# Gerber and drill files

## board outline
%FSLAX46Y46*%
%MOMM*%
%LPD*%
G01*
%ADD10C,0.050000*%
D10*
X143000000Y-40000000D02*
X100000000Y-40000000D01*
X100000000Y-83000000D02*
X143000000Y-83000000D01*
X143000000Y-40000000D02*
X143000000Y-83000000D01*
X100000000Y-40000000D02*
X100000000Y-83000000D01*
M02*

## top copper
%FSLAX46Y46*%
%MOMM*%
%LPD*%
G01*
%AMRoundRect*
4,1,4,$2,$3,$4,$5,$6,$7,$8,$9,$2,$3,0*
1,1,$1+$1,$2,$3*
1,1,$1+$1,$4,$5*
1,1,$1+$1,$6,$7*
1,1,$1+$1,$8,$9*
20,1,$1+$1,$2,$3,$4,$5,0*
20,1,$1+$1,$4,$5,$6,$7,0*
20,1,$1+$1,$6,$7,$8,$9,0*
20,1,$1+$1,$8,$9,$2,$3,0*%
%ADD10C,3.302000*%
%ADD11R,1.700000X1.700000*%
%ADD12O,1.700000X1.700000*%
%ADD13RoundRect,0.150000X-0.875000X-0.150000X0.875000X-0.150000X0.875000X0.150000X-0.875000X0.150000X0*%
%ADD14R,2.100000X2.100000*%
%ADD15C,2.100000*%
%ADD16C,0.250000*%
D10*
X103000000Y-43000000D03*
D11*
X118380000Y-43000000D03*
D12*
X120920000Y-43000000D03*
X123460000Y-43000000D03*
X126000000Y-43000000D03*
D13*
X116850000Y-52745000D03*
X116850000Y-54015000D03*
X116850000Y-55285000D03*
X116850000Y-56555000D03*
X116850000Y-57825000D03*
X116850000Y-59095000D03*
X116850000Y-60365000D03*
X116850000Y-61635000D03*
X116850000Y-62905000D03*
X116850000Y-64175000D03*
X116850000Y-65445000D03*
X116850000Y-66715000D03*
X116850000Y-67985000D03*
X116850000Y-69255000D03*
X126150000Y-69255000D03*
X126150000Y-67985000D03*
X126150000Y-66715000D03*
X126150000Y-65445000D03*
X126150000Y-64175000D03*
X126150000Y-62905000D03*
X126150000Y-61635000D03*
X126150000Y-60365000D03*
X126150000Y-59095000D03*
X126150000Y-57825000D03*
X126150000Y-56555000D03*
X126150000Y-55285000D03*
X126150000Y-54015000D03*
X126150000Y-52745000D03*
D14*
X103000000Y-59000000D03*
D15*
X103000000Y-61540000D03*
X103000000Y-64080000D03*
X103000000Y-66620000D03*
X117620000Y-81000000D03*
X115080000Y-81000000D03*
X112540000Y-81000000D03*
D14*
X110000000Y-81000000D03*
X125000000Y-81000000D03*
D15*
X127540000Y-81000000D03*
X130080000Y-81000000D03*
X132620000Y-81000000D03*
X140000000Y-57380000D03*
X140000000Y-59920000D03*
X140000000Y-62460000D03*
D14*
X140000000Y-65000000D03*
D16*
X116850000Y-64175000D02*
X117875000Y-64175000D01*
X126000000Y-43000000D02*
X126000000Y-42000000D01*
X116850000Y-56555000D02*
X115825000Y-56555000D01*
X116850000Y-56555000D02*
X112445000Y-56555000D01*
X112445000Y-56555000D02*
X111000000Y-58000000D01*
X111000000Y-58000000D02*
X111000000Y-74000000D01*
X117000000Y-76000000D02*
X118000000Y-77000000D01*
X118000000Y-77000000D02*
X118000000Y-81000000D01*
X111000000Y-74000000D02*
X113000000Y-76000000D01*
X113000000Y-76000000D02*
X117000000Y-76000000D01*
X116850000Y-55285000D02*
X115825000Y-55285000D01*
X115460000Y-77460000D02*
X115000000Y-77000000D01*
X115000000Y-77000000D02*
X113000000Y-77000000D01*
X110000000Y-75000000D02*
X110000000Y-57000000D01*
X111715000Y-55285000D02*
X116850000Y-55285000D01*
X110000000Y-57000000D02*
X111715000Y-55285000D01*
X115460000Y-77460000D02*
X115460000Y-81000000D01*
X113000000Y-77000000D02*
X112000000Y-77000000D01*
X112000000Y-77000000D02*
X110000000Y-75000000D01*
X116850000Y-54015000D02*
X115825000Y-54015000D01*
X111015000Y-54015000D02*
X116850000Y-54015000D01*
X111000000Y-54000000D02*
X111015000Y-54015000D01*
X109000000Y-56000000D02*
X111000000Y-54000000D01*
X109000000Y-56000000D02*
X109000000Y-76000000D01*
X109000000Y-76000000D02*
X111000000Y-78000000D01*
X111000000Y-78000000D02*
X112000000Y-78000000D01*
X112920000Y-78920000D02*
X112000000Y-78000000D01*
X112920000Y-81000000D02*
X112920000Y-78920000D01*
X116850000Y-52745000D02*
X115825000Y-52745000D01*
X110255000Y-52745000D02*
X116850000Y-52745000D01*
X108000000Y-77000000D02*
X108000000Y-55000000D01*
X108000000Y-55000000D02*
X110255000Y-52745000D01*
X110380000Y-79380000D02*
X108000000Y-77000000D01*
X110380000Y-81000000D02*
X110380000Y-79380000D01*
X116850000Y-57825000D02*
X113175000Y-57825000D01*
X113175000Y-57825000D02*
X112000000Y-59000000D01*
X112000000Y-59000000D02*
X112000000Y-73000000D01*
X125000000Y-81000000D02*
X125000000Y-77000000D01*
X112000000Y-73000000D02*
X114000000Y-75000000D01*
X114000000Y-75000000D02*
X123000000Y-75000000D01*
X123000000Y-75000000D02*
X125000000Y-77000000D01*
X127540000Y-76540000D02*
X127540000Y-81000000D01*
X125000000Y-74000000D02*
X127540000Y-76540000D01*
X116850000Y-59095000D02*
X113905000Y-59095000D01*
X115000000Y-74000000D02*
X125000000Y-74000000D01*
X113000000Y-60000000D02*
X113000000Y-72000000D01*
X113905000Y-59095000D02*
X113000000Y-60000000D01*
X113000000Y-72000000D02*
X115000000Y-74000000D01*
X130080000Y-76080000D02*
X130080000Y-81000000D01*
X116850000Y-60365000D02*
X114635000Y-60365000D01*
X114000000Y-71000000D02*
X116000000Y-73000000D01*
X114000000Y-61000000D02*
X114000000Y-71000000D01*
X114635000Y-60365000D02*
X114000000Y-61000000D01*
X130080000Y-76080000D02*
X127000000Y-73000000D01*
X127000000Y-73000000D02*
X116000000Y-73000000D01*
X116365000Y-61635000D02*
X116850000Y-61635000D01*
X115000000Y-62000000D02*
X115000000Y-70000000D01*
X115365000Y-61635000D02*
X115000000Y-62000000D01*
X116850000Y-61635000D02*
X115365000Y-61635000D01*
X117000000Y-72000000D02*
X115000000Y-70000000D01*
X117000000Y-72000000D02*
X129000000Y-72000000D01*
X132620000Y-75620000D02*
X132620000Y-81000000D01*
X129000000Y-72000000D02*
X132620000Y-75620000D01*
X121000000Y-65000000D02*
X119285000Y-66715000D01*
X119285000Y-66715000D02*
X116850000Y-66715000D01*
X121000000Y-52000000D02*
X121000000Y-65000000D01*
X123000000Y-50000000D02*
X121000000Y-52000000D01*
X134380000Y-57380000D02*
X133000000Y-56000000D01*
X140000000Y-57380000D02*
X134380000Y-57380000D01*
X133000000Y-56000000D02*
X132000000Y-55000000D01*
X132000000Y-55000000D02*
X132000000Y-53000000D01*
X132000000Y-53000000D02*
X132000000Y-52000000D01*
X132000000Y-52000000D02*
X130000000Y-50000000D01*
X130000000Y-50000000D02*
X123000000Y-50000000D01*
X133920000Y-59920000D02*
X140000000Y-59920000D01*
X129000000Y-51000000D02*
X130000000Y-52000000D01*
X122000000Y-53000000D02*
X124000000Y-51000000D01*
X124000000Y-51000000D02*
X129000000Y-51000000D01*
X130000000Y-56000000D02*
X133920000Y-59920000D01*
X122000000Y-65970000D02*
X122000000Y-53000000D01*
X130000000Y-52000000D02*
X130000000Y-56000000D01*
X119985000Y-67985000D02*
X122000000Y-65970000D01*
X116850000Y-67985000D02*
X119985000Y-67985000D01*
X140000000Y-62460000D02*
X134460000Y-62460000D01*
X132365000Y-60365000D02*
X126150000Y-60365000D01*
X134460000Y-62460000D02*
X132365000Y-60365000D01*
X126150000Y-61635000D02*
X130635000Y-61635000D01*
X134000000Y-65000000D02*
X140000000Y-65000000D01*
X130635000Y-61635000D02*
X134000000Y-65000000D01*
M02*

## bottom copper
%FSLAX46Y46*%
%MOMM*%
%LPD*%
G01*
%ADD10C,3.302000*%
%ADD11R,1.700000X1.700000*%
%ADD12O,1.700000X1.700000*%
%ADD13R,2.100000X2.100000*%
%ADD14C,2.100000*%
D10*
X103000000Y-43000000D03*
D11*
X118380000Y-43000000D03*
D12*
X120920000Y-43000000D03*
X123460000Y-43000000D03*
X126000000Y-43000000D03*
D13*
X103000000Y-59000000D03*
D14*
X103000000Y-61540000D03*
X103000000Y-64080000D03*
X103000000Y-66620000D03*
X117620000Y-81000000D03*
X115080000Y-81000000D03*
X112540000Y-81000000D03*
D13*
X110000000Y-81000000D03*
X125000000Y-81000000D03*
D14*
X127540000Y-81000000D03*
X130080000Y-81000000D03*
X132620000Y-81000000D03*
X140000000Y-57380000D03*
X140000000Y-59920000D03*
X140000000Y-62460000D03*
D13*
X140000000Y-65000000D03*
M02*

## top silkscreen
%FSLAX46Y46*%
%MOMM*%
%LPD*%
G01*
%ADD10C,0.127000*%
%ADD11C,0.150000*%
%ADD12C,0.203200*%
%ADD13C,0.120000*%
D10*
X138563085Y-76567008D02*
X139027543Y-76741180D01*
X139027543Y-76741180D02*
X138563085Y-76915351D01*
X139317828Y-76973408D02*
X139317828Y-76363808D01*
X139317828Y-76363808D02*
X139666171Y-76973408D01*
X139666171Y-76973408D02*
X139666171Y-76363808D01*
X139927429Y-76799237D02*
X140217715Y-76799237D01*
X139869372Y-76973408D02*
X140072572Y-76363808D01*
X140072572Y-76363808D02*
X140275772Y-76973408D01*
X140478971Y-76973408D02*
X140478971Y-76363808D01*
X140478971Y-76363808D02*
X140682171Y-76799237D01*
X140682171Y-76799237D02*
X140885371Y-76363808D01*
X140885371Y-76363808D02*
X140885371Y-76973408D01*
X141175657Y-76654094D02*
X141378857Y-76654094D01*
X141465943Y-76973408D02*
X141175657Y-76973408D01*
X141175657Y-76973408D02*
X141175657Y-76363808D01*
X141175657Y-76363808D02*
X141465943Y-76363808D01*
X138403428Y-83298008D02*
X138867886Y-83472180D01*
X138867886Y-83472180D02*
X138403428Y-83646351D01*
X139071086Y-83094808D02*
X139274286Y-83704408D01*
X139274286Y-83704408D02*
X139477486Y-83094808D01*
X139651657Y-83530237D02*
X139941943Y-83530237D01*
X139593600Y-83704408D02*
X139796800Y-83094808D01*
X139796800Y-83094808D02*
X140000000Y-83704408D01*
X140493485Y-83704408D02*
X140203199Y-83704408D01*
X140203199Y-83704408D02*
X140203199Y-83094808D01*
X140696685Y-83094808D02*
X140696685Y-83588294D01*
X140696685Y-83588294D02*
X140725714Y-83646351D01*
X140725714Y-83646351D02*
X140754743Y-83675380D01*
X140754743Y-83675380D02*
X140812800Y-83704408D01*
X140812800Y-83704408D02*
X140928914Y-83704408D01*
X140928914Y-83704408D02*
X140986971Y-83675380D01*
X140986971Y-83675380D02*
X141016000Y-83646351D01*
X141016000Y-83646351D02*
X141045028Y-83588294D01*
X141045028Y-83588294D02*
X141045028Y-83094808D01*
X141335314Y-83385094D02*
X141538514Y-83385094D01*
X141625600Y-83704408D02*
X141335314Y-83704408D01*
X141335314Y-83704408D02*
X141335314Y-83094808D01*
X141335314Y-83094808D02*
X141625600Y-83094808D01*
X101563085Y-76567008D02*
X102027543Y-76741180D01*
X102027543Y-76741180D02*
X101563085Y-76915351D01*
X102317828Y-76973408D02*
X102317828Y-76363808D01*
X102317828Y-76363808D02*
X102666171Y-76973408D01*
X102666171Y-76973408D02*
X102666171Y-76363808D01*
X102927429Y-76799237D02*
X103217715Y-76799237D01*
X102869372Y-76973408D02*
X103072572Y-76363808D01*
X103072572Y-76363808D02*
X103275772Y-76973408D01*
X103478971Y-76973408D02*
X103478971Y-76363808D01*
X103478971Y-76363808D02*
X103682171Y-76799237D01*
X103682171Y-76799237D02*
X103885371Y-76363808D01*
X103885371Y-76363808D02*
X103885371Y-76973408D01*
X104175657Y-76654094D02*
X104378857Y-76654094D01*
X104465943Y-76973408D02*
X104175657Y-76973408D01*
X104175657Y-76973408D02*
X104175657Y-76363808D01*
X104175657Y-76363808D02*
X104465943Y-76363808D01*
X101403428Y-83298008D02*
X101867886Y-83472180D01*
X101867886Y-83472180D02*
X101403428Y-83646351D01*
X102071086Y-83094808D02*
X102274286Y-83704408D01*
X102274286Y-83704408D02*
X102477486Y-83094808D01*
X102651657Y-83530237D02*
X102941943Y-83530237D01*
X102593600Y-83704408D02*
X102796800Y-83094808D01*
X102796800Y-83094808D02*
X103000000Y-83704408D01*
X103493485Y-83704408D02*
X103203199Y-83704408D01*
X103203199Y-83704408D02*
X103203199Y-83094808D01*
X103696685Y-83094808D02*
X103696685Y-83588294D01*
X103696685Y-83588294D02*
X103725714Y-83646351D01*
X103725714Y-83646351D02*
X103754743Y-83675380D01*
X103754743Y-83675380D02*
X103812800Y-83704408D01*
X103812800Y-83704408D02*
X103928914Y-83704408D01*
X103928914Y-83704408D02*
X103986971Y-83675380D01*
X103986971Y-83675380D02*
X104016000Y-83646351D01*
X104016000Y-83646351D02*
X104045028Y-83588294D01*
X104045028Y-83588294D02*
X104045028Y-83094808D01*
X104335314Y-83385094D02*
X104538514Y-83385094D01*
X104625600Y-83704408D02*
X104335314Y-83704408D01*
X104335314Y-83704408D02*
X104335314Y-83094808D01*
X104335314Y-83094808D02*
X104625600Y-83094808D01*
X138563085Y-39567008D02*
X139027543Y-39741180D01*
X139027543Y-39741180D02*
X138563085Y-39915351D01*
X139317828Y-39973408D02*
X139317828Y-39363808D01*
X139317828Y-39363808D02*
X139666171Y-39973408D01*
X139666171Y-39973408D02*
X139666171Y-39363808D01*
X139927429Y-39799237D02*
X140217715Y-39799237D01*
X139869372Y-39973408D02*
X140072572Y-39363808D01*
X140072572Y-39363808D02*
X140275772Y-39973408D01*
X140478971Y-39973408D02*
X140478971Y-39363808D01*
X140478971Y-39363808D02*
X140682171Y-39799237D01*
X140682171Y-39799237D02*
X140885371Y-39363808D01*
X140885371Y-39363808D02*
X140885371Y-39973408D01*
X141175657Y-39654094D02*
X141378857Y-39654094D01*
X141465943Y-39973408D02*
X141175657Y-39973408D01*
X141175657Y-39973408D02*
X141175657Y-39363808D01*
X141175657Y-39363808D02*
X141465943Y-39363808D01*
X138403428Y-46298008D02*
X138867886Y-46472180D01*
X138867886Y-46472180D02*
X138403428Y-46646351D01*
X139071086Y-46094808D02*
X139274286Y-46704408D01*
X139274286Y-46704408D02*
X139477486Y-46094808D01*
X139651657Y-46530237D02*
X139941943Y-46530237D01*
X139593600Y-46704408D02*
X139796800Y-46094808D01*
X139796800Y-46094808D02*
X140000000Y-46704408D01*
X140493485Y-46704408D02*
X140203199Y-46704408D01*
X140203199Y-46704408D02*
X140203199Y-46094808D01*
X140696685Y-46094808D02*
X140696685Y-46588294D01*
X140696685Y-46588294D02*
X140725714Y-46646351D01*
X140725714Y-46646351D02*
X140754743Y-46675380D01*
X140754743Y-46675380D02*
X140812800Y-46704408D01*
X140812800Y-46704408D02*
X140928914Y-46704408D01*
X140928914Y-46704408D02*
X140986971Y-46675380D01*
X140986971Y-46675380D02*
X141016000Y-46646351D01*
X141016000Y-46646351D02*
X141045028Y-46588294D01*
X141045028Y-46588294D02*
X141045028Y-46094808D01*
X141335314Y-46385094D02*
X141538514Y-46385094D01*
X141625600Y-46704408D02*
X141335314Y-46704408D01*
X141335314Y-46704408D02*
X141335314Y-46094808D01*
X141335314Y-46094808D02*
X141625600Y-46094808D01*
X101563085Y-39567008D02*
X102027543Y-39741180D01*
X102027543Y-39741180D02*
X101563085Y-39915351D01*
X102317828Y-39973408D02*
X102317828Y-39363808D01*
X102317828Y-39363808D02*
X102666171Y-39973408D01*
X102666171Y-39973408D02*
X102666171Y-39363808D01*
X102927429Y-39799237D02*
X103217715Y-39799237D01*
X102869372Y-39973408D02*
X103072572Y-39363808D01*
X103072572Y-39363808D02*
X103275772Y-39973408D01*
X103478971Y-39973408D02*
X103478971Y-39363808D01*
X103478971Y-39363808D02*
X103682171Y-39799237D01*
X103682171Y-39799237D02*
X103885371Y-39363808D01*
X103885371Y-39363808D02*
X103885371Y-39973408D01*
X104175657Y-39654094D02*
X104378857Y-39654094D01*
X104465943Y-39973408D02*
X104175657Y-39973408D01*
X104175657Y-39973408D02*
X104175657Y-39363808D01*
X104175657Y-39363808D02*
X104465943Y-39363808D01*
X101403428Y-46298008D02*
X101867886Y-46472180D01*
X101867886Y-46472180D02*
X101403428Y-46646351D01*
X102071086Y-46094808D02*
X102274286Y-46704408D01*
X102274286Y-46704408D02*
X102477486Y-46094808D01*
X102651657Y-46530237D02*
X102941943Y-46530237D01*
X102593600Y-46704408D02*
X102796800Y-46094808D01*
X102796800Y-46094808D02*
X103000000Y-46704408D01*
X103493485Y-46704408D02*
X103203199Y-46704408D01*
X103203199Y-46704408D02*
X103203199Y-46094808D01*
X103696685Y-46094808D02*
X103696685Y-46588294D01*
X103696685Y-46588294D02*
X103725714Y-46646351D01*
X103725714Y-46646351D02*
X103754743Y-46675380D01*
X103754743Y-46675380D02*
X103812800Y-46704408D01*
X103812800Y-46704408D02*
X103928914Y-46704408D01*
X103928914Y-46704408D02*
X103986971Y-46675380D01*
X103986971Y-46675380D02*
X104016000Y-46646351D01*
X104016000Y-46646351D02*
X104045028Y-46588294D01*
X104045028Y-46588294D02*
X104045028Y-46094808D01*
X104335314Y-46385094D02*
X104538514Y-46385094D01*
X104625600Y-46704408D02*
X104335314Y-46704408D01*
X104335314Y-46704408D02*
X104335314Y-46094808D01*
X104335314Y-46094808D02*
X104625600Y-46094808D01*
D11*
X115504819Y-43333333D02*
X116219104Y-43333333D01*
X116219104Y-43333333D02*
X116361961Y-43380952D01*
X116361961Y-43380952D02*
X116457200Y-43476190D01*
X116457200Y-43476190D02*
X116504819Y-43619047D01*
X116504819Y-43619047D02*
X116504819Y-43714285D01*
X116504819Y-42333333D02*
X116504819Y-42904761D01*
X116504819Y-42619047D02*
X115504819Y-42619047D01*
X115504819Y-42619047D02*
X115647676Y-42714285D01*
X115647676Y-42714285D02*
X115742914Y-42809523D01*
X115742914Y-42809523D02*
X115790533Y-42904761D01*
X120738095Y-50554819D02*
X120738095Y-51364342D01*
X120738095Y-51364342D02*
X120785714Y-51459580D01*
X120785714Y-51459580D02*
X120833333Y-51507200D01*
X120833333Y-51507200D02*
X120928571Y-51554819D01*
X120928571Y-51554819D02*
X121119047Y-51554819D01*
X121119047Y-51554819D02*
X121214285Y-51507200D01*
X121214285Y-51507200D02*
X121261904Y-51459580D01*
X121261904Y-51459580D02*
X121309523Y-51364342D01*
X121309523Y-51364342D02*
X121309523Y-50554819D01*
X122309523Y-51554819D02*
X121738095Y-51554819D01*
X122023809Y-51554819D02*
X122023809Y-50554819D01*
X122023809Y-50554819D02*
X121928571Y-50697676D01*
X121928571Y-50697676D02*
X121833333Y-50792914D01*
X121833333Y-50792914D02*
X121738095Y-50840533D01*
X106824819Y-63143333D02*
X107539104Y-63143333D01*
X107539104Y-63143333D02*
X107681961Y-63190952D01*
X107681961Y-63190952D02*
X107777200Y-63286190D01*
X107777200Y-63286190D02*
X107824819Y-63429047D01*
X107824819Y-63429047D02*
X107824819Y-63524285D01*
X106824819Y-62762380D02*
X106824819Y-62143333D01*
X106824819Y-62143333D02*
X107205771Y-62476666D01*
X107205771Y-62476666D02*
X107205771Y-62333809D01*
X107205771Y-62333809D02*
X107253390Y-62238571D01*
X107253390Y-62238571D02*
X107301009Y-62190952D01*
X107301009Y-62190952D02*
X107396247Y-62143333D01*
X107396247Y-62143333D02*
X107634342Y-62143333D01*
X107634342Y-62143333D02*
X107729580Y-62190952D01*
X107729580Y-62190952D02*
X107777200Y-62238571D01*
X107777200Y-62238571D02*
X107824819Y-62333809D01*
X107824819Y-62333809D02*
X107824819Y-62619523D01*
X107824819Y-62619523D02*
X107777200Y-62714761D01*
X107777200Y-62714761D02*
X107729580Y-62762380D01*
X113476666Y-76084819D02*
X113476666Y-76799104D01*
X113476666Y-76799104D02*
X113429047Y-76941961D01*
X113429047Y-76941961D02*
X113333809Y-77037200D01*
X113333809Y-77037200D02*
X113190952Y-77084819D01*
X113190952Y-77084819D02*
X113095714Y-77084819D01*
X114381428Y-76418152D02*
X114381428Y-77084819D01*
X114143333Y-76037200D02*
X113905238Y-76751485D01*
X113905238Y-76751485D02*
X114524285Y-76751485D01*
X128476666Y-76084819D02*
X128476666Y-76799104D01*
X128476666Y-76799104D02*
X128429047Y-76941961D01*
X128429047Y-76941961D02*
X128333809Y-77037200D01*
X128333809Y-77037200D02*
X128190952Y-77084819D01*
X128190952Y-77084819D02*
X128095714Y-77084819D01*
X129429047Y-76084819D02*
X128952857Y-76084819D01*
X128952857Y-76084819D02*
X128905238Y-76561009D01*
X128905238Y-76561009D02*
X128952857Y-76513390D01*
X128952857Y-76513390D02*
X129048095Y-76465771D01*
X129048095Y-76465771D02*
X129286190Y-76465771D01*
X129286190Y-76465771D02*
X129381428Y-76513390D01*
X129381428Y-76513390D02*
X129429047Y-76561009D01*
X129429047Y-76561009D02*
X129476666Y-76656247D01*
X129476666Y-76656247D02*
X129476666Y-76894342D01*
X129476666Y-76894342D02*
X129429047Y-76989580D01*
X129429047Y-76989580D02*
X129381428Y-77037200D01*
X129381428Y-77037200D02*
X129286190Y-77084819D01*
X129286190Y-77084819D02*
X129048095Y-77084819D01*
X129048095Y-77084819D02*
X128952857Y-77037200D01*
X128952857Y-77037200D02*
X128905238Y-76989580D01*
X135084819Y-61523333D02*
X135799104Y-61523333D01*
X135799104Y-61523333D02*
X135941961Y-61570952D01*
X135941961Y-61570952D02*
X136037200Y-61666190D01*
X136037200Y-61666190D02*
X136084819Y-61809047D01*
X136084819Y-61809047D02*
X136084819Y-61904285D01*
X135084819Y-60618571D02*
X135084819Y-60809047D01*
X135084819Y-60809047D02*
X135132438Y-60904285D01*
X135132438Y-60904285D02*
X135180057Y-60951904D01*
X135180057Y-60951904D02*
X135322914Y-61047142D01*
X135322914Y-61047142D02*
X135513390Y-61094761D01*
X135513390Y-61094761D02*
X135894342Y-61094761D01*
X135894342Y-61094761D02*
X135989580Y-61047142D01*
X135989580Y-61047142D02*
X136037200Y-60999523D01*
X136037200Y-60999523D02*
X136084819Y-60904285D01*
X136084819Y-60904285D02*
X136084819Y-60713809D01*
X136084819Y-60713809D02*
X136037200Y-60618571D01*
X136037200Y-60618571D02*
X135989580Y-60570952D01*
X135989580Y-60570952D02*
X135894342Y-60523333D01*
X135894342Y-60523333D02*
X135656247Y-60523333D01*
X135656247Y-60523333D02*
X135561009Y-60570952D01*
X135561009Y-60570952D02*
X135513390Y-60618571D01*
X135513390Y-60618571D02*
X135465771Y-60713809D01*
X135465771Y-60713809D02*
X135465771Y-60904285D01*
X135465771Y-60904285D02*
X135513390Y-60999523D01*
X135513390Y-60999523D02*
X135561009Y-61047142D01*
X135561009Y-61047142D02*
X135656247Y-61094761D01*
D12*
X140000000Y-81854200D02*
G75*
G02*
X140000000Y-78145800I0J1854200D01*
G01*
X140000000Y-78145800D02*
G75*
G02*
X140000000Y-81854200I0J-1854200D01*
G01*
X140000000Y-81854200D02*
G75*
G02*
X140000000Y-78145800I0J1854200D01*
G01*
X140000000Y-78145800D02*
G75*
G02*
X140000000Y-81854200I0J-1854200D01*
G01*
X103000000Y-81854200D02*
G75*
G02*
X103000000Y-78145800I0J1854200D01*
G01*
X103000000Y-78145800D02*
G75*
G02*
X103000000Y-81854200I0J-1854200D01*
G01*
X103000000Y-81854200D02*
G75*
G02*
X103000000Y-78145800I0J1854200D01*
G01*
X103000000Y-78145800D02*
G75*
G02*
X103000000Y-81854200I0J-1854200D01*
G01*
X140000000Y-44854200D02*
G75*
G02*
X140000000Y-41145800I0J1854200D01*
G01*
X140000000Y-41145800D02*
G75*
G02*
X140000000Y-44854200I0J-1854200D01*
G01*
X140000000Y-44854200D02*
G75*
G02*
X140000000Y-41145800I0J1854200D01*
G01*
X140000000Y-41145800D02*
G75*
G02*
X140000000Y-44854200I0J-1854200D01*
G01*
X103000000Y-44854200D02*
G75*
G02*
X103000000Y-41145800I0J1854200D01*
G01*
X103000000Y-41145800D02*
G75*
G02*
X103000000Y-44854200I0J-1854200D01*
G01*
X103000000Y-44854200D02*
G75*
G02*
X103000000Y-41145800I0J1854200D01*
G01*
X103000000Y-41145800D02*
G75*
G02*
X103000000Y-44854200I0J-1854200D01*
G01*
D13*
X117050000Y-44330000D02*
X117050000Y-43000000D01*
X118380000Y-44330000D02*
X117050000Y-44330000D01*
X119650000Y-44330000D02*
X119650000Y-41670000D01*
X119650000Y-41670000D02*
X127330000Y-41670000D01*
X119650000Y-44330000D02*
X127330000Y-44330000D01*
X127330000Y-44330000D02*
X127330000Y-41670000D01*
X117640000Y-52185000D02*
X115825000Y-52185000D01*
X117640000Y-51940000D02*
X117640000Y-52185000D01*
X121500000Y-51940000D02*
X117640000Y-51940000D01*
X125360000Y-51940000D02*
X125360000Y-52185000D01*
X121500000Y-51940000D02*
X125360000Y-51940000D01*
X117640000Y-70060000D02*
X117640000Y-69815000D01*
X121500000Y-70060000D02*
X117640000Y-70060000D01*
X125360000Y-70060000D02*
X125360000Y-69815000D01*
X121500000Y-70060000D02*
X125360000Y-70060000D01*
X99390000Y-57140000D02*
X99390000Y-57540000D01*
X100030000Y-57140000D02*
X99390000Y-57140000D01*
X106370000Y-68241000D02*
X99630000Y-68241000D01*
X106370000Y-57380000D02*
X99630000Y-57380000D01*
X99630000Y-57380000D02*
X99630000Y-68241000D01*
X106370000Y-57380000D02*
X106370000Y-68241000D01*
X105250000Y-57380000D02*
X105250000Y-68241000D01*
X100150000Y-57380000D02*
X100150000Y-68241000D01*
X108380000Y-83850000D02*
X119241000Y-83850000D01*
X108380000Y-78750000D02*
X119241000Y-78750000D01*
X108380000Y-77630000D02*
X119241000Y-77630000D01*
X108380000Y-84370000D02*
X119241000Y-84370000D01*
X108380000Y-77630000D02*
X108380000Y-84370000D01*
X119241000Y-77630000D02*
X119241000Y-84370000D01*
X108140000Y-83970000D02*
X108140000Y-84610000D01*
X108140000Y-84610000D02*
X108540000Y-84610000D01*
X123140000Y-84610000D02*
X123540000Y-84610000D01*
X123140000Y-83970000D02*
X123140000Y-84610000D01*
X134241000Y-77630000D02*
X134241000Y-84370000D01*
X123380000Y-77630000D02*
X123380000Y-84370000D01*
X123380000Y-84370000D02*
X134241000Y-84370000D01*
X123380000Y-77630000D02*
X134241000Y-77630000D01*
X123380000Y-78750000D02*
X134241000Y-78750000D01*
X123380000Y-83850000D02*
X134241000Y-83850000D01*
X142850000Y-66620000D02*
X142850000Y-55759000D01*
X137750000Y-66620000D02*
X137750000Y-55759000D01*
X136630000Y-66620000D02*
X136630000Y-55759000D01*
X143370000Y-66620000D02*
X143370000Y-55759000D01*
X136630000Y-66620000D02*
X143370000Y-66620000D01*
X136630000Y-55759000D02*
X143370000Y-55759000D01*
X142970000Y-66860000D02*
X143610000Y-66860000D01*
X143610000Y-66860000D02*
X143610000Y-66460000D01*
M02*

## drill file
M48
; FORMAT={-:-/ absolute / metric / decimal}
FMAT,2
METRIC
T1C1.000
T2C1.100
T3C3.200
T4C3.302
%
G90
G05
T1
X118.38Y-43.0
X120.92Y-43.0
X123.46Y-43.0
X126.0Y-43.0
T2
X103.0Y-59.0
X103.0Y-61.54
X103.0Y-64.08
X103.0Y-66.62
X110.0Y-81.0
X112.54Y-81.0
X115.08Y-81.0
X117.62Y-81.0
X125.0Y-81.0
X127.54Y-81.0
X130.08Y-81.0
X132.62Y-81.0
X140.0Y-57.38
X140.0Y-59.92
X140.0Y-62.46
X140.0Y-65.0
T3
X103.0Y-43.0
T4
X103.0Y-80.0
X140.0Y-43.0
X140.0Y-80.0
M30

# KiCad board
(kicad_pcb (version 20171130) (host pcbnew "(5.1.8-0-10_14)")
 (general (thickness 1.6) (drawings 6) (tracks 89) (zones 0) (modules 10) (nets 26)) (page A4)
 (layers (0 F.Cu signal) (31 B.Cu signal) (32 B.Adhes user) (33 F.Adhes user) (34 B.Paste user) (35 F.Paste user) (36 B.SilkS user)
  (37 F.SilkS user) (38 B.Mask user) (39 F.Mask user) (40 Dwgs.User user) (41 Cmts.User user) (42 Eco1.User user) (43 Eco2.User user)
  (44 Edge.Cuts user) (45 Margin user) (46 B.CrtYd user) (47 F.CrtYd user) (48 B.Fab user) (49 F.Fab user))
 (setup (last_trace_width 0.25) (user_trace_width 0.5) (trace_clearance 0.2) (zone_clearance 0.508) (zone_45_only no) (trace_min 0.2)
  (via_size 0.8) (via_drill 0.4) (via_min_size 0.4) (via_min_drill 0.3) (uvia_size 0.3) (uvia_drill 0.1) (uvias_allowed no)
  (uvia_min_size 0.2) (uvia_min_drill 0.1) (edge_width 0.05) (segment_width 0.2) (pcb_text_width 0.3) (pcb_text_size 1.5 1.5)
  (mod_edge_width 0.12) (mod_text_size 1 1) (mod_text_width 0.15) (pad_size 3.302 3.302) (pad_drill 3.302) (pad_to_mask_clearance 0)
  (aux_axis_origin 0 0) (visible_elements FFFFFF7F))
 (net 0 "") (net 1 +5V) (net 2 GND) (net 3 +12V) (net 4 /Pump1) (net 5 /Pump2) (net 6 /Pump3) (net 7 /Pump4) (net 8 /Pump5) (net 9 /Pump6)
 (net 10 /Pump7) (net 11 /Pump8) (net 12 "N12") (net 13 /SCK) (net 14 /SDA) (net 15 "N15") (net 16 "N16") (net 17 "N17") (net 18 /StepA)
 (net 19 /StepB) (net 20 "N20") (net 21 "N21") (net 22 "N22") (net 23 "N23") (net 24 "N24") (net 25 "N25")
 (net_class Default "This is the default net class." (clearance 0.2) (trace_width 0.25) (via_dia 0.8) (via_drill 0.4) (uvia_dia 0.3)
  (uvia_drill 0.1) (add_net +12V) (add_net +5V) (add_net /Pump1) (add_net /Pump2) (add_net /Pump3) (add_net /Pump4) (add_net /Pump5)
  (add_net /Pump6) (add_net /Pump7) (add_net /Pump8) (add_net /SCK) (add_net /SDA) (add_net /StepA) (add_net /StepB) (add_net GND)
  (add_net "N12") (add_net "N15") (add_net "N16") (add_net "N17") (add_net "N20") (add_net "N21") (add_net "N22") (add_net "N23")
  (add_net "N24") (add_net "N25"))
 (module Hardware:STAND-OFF (layer F.Cu) (at 140 80)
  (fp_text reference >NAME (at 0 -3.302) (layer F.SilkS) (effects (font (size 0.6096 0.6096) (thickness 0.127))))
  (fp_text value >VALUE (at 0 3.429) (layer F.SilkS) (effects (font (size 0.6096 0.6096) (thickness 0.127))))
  (fp_arc (start 0 0) (end 0 1.8542) (angle 180) (layer F.SilkS) (width 0.2032))
  (fp_arc (start 0 0) (end 0 -1.8542) (angle 180) (layer F.SilkS) (width 0.2032))
  (fp_arc (start 0 0) (end 0 1.8542) (angle 180) (layer F.SilkS) (width 0.2032))
  (fp_arc (start 0 0) (end 0 -1.8542) (angle 180) (layer F.SilkS) (width 0.2032))
  (pad "" np_thru_hole circle (at 0 0) (size 3.302 3.302) (drill 3.302) (layers *.Cu *.Mask) (solder_mask_margin 0.1016)))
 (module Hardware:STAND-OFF (layer F.Cu) (at 103 80)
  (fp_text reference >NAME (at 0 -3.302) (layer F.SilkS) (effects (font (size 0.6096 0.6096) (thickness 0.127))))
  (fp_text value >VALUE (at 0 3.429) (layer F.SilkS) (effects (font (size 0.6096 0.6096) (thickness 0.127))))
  (fp_arc (start 0 0) (end 0 1.8542) (angle 180) (layer F.SilkS) (width 0.2032))
  (fp_arc (start 0 0) (end 0 -1.8542) (angle 180) (layer F.SilkS) (width 0.2032))
  (fp_arc (start 0 0) (end 0 1.8542) (angle 180) (layer F.SilkS) (width 0.2032))
  (fp_arc (start 0 0) (end 0 -1.8542) (angle 180) (layer F.SilkS) (width 0.2032))
  (pad "" np_thru_hole circle (at 0 0) (size 3.302 3.302) (drill 3.302) (layers *.Cu *.Mask) (solder_mask_margin 0.1016)))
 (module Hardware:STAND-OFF (layer F.Cu) (at 140 43)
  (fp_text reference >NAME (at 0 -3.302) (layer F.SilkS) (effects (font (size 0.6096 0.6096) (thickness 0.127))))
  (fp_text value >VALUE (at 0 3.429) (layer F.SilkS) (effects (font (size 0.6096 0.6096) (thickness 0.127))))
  (fp_arc (start 0 0) (end 0 1.8542) (angle 180) (layer F.SilkS) (width 0.2032))
  (fp_arc (start 0 0) (end 0 -1.8542) (angle 180) (layer F.SilkS) (width 0.2032))
  (fp_arc (start 0 0) (end 0 1.8542) (angle 180) (layer F.SilkS) (width 0.2032))
  (fp_arc (start 0 0) (end 0 -1.8542) (angle 180) (layer F.SilkS) (width 0.2032))
  (pad "" np_thru_hole circle (at 0 0) (size 3.302 3.302) (drill 3.302) (layers *.Cu *.Mask) (solder_mask_margin 0.1016)))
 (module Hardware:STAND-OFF (layer F.Cu) (at 103 43)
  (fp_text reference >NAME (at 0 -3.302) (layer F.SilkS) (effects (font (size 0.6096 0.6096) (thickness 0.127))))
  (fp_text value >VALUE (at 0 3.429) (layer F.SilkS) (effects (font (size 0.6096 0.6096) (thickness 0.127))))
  (fp_arc (start 0 0) (end 0 1.8542) (angle 180) (layer F.SilkS) (width 0.2032))
  (fp_arc (start 0 0) (end 0 -1.8542) (angle 180) (layer F.SilkS) (width 0.2032))
  (fp_arc (start 0 0) (end 0 1.8542) (angle 180) (layer F.SilkS) (width 0.2032))
  (fp_arc (start 0 0) (end 0 -1.8542) (angle 180) (layer F.SilkS) (width 0.2032))
  (pad "" np_thru_hole circle (at 0 0) (size 3.302 3.302) (drill 3.2) (layers *.Cu *.Mask) (solder_mask_margin 0.1016)))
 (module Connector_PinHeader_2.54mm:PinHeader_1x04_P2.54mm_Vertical (layer F.Cu) (at 118.38 43 90)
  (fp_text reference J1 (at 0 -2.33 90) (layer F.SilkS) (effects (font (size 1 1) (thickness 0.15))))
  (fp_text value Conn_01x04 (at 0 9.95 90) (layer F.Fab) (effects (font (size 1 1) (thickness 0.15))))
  (fp_line (start -1.33 -1.33) (end 0 -1.33) (layer F.SilkS) (width 0.12))
  (fp_line (start -1.33 0) (end -1.33 -1.33) (layer F.SilkS) (width 0.12))
  (fp_line (start -1.33 1.27) (end 1.33 1.27) (layer F.SilkS) (width 0.12))
  (fp_line (start 1.33 1.27) (end 1.33 8.95) (layer F.SilkS) (width 0.12))
  (fp_line (start -1.33 1.27) (end -1.33 8.95) (layer F.SilkS) (width 0.12))
  (fp_line (start -1.33 8.95) (end 1.33 8.95) (layer F.SilkS) (width 0.12))
  (pad 1 thru_hole rect (at 0 0 90) (size 1.7 1.7) (drill 1) (layers *.Cu *.Mask) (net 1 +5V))
  (pad 2 thru_hole oval (at 0 2.54 90) (size 1.7 1.7) (drill 1) (layers *.Cu *.Mask) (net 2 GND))
  (pad 3 thru_hole oval (at 0 5.08 90) (size 1.7 1.7) (drill 1) (layers *.Cu *.Mask) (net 2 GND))
  (pad 4 thru_hole oval (at 0 7.62 90) (size 1.7 1.7) (drill 1) (layers *.Cu *.Mask) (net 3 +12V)))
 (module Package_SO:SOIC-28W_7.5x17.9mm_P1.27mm (layer F.Cu) (at 121.5 61)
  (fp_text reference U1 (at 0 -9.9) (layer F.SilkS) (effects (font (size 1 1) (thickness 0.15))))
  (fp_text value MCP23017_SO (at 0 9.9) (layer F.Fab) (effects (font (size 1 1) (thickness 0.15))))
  (fp_line (start -3.86 -8.815) (end -5.675 -8.815) (layer F.SilkS) (width 0.12))
  (fp_line (start -3.86 -9.06) (end -3.86 -8.815) (layer F.SilkS) (width 0.12))
  (fp_line (start 0 -9.06) (end -3.86 -9.06) (layer F.SilkS) (width 0.12))
  (fp_line (start 3.86 -9.06) (end 3.86 -8.815) (layer F.SilkS) (width 0.12))
  (fp_line (start 0 -9.06) (end 3.86 -9.06) (layer F.SilkS) (width 0.12))
  (fp_line (start -3.86 9.06) (end -3.86 8.815) (layer F.SilkS) (width 0.12))
  (fp_line (start 0 9.06) (end -3.86 9.06) (layer F.SilkS) (width 0.12))
  (fp_line (start 3.86 9.06) (end 3.86 8.815) (layer F.SilkS) (width 0.12))
  (fp_line (start 0 9.06) (end 3.86 9.06) (layer F.SilkS) (width 0.12))
  (pad 1 smd roundrect (at -4.65 -8.255) (size 2.05 0.6) (layers F.Cu F.Paste F.Mask) (roundrect_rratio 0.25) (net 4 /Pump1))
  (pad 2 smd roundrect (at -4.65 -6.985) (size 2.05 0.6) (layers F.Cu F.Paste F.Mask) (roundrect_rratio 0.25) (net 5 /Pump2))
  (pad 3 smd roundrect (at -4.65 -5.715) (size 2.05 0.6) (layers F.Cu F.Paste F.Mask) (roundrect_rratio 0.25) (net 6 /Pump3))
  (pad 4 smd roundrect (at -4.65 -4.445) (size 2.05 0.6) (layers F.Cu F.Paste F.Mask) (roundrect_rratio 0.25) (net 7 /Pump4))
  (pad 5 smd roundrect (at -4.65 -3.175) (size 2.05 0.6) (layers F.Cu F.Paste F.Mask) (roundrect_rratio 0.25) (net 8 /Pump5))
  (pad 6 smd roundrect (at -4.65 -1.905) (size 2.05 0.6) (layers F.Cu F.Paste F.Mask) (roundrect_rratio 0.25) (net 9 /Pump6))
  (pad 7 smd roundrect (at -4.65 -0.635) (size 2.05 0.6) (layers F.Cu F.Paste F.Mask) (roundrect_rratio 0.25) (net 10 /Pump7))
  (pad 8 smd roundrect (at -4.65 0.635) (size 2.05 0.6) (layers F.Cu F.Paste F.Mask) (roundrect_rratio 0.25) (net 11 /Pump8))
  (pad 9 smd roundrect (at -4.65 1.905) (size 2.05 0.6) (layers F.Cu F.Paste F.Mask) (roundrect_rratio 0.25) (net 1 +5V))
  (pad 10 smd roundrect (at -4.65 3.175) (size 2.05 0.6) (layers F.Cu F.Paste F.Mask) (roundrect_rratio 0.25) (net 2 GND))
  (pad 11 smd roundrect (at -4.65 4.445) (size 2.05 0.6) (layers F.Cu F.Paste F.Mask) (roundrect_rratio 0.25) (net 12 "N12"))
  (pad 12 smd roundrect (at -4.65 5.715) (size 2.05 0.6) (layers F.Cu F.Paste F.Mask) (roundrect_rratio 0.25) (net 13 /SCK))
  (pad 13 smd roundrect (at -4.65 6.985) (size 2.05 0.6) (layers F.Cu F.Paste F.Mask) (roundrect_rratio 0.25) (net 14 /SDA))
  (pad 14 smd roundrect (at -4.65 8.255) (size 2.05 0.6) (layers F.Cu F.Paste F.Mask) (roundrect_rratio 0.25) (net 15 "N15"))
  (pad 15 smd roundrect (at 4.65 8.255) (size 2.05 0.6) (layers F.Cu F.Paste F.Mask) (roundrect_rratio 0.25) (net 2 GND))
  (pad 16 smd roundrect (at 4.65 6.985) (size 2.05 0.6) (layers F.Cu F.Paste F.Mask) (roundrect_rratio 0.25) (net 2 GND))
  (pad 17 smd roundrect (at 4.65 5.715) (size 2.05 0.6) (layers F.Cu F.Paste F.Mask) (roundrect_rratio 0.25) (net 2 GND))
  (pad 18 smd roundrect (at 4.65 4.445) (size 2.05 0.6) (layers F.Cu F.Paste F.Mask) (roundrect_rratio 0.25) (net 1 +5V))
  (pad 19 smd roundrect (at 4.65 3.175) (size 2.05 0.6) (layers F.Cu F.Paste F.Mask) (roundrect_rratio 0.25) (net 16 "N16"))
  (pad 20 smd roundrect (at 4.65 1.905) (size 2.05 0.6) (layers F.Cu F.Paste F.Mask) (roundrect_rratio 0.25) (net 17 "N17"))
  (pad 21 smd roundrect (at 4.65 0.635) (size 2.05 0.6) (layers F.Cu F.Paste F.Mask) (roundrect_rratio 0.25) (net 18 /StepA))
  (pad 22 smd roundrect (at 4.65 -0.635) (size 2.05 0.6) (layers F.Cu F.Paste F.Mask) (roundrect_rratio 0.25) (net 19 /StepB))
  (pad 23 smd roundrect (at 4.65 -1.905) (size 2.05 0.6) (layers F.Cu F.Paste F.Mask) (roundrect_rratio 0.25) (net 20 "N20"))
  (pad 24 smd roundrect (at 4.65 -3.175) (size 2.05 0.6) (layers F.Cu F.Paste F.Mask) (roundrect_rratio 0.25) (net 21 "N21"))
  (pad 25 smd roundrect (at 4.65 -4.445) (size 2.05 0.6) (layers F.Cu F.Paste F.Mask) (roundrect_rratio 0.25) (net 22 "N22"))
  (pad 26 smd roundrect (at 4.65 -5.715) (size 2.05 0.6) (layers F.Cu F.Paste F.Mask) (roundrect_rratio 0.25) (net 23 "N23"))
  (pad 27 smd roundrect (at 4.65 -6.985) (size 2.05 0.6) (layers F.Cu F.Paste F.Mask) (roundrect_rratio 0.25) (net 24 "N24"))
  (pad 28 smd roundrect (at 4.65 -8.255) (size 2.05 0.6) (layers F.Cu F.Paste F.Mask) (roundrect_rratio 0.25) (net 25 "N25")))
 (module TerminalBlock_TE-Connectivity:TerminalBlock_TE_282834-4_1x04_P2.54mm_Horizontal (layer F.Cu) (at 103 59 270)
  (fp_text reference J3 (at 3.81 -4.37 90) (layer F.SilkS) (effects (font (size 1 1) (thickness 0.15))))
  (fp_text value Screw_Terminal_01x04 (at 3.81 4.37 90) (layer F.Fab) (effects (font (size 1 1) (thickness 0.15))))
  (fp_line (start -1.86 3.61) (end -1.46 3.61) (layer F.SilkS) (width 0.12))
  (fp_line (start -1.86 2.97) (end -1.86 3.61) (layer F.SilkS) (width 0.12))
  (fp_line (start 9.241 -3.37) (end 9.241 3.37) (layer F.SilkS) (width 0.12))
  (fp_line (start -1.62 -3.37) (end -1.62 3.37) (layer F.SilkS) (width 0.12))
  (fp_line (start -1.62 3.37) (end 9.241 3.37) (layer F.SilkS) (width 0.12))
  (fp_line (start -1.62 -3.37) (end 9.241 -3.37) (layer F.SilkS) (width 0.12))
  (fp_line (start -1.62 -2.25) (end 9.241 -2.25) (layer F.SilkS) (width 0.12))
  (fp_line (start -1.62 2.85) (end 9.241 2.85) (layer F.SilkS) (width 0.12))
  (pad 1 thru_hole rect (at 0 0 270) (size 2.1 2.1) (drill 1.1) (layers *.Cu *.Mask) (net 1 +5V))
  (pad 2 thru_hole circle (at 2.54 0 270) (size 2.1 2.1) (drill 1.1) (layers *.Cu *.Mask) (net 2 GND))
  (pad 3 thru_hole circle (at 5.08 0 270) (size 2.1 2.1) (drill 1.1) (layers *.Cu *.Mask) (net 2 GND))
  (pad 4 thru_hole circle (at 7.62 0 270) (size 2.1 2.1) (drill 1.1) (layers *.Cu *.Mask) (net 3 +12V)))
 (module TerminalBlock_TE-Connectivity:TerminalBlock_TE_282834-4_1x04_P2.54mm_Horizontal (layer F.Cu) (at 110 81)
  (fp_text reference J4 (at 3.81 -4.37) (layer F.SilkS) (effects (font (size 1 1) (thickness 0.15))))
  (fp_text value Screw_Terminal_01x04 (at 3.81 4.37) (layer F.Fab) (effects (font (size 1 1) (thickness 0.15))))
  (fp_line (start -1.62 2.85) (end 9.241 2.85) (layer F.SilkS) (width 0.12))
  (fp_line (start -1.62 -2.25) (end 9.241 -2.25) (layer F.SilkS) (width 0.12))
  (fp_line (start -1.62 -3.37) (end 9.241 -3.37) (layer F.SilkS) (width 0.12))
  (fp_line (start -1.62 3.37) (end 9.241 3.37) (layer F.SilkS) (width 0.12))
  (fp_line (start -1.62 -3.37) (end -1.62 3.37) (layer F.SilkS) (width 0.12))
  (fp_line (start 9.241 -3.37) (end 9.241 3.37) (layer F.SilkS) (width 0.12))
  (fp_line (start -1.86 2.97) (end -1.86 3.61) (layer F.SilkS) (width 0.12))
  (fp_line (start -1.86 3.61) (end -1.46 3.61) (layer F.SilkS) (width 0.12))
  (pad 4 thru_hole circle (at 7.62 0) (size 2.1 2.1) (drill 1.1) (layers *.Cu *.Mask) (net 7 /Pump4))
  (pad 3 thru_hole circle (at 5.08 0) (size 2.1 2.1) (drill 1.1) (layers *.Cu *.Mask) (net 6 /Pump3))
  (pad 2 thru_hole circle (at 2.54 0) (size 2.1 2.1) (drill 1.1) (layers *.Cu *.Mask) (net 5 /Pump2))
  (pad 1 thru_hole rect (at 0 0) (size 2.1 2.1) (drill 1.1) (layers *.Cu *.Mask) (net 4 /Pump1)))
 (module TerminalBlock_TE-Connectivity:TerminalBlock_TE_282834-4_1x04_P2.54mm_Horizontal (layer F.Cu) (at 125 81)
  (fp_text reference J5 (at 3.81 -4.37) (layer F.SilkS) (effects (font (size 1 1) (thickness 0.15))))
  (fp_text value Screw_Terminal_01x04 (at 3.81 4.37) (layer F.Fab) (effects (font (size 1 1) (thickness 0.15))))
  (fp_line (start -1.86 3.61) (end -1.46 3.61) (layer F.SilkS) (width 0.12))
  (fp_line (start -1.86 2.97) (end -1.86 3.61) (layer F.SilkS) (width 0.12))
  (fp_line (start 9.241 -3.37) (end 9.241 3.37) (layer F.SilkS) (width 0.12))
  (fp_line (start -1.62 -3.37) (end -1.62 3.37) (layer F.SilkS) (width 0.12))
  (fp_line (start -1.62 3.37) (end 9.241 3.37) (layer F.SilkS) (width 0.12))
  (fp_line (start -1.62 -3.37) (end 9.241 -3.37) (layer F.SilkS) (width 0.12))
  (fp_line (start -1.62 -2.25) (end 9.241 -2.25) (layer F.SilkS) (width 0.12))
  (fp_line (start -1.62 2.85) (end 9.241 2.85) (layer F.SilkS) (width 0.12))
  (pad 1 thru_hole rect (at 0 0) (size 2.1 2.1) (drill 1.1) (layers *.Cu *.Mask) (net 8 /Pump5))
  (pad 2 thru_hole circle (at 2.54 0) (size 2.1 2.1) (drill 1.1) (layers *.Cu *.Mask) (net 9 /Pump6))
  (pad 3 thru_hole circle (at 5.08 0) (size 2.1 2.1) (drill 1.1) (layers *.Cu *.Mask) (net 10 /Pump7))
  (pad 4 thru_hole circle (at 7.62 0) (size 2.1 2.1) (drill 1.1) (layers *.Cu *.Mask) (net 11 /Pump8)))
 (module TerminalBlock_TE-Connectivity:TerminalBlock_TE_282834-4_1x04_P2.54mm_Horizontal (layer F.Cu) (at 140 65 90)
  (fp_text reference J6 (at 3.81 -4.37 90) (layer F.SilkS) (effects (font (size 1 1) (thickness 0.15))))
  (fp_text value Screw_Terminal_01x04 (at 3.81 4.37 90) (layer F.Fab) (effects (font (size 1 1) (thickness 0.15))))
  (fp_line (start -1.62 2.85) (end 9.241 2.85) (layer F.SilkS) (width 0.12))
  (fp_line (start -1.62 -2.25) (end 9.241 -2.25) (layer F.SilkS) (width 0.12))
  (fp_line (start -1.62 -3.37) (end 9.241 -3.37) (layer F.SilkS) (width 0.12))
  (fp_line (start -1.62 3.37) (end 9.241 3.37) (layer F.SilkS) (width 0.12))
  (fp_line (start -1.62 -3.37) (end -1.62 3.37) (layer F.SilkS) (width 0.12))
  (fp_line (start 9.241 -3.37) (end 9.241 3.37) (layer F.SilkS) (width 0.12))
  (fp_line (start -1.86 2.97) (end -1.86 3.61) (layer F.SilkS) (width 0.12))
  (fp_line (start -1.86 3.61) (end -1.46 3.61) (layer F.SilkS) (width 0.12))
  (pad 4 thru_hole circle (at 7.62 0 90) (size 2.1 2.1) (drill 1.1) (layers *.Cu *.Mask) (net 13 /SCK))
  (pad 3 thru_hole circle (at 5.08 0 90) (size 2.1 2.1) (drill 1.1) (layers *.Cu *.Mask) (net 14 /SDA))
  (pad 2 thru_hole circle (at 2.54 0 90) (size 2.1 2.1) (drill 1.1) (layers *.Cu *.Mask) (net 19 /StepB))
  (pad 1 thru_hole rect (at 0 0 90) (size 2.1 2.1) (drill 1.1) (layers *.Cu *.Mask) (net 18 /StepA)))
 (gr_line (start 143 40) (end 100 40) (layer Edge.Cuts) (width 0.05))
 (gr_line (start 100 83) (end 143 83) (layer Edge.Cuts) (width 0.05))
 (gr_line (start 143 40) (end 143 83) (layer Edge.Cuts) (width 0.05))
 (gr_line (start 100 40) (end 100 83) (layer Edge.Cuts) (width 0.05))
 (segment (start 116.85 64.175) (end 117.875 64.175) (width 0.25) (layer F.Cu) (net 2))
 (segment (start 126 43) (end 126 42) (width 0.25) (layer F.Cu) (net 3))
 (segment (start 116.85 56.555) (end 115.825 56.555) (width 0.25) (layer F.Cu) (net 7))
 (segment (start 116.85 56.555) (end 112.445 56.555) (width 0.25) (layer F.Cu) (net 7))
 (segment (start 112.445 56.555) (end 111 58) (width 0.25) (layer F.Cu) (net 7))
 (segment (start 111 58) (end 111 74) (width 0.25) (layer F.Cu) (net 7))
 (segment (start 117 76) (end 118 77) (width 0.25) (layer F.Cu) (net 7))
 (segment (start 118 77) (end 118 81) (width 0.25) (layer F.Cu) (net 7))
 (segment (start 111 74) (end 113 76) (width 0.25) (layer F.Cu) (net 7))
 (segment (start 113 76) (end 117 76) (width 0.25) (layer F.Cu) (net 7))
 (segment (start 116.85 55.285) (end 115.825 55.285) (width 0.25) (layer F.Cu) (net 6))
 (segment (start 115.46 77.46) (end 115 77) (width 0.25) (layer F.Cu) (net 6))
 (segment (start 115 77) (end 113 77) (width 0.25) (layer F.Cu) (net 6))
 (segment (start 110 75) (end 110 57) (width 0.25) (layer F.Cu) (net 6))
 (segment (start 111.715 55.285) (end 116.85 55.285) (width 0.25) (layer F.Cu) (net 6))
 (segment (start 110 57) (end 111.715 55.285) (width 0.25) (layer F.Cu) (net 6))
 (segment (start 115.46 77.46) (end 115.46 81) (width 0.25) (layer F.Cu) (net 6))
 (segment (start 113 77) (end 112 77) (width 0.25) (layer F.Cu) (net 6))
 (segment (start 112 77) (end 110 75) (width 0.25) (layer F.Cu) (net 6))
 (segment (start 116.85 54.015) (end 115.825 54.015) (width 0.25) (layer F.Cu) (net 5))
 (segment (start 111.015 54.015) (end 116.85 54.015) (width 0.25) (layer F.Cu) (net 5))
 (segment (start 111 54) (end 111.015 54.015) (width 0.25) (layer F.Cu) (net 5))
 (segment (start 109 56) (end 111 54) (width 0.25) (layer F.Cu) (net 5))
 (segment (start 109 56) (end 109 76) (width 0.25) (layer F.Cu) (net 5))
 (segment (start 109 76) (end 111 78) (width 0.25) (layer F.Cu) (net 5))
 (segment (start 111 78) (end 112 78) (width 0.25) (layer F.Cu) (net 5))
 (segment (start 112.92 78.92) (end 112 78) (width 0.25) (layer F.Cu) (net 5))
 (segment (start 112.92 81) (end 112.92 78.92) (width 0.25) (layer F.Cu) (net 5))
 (segment (start 116.85 52.745) (end 115.825 52.745) (width 0.25) (layer F.Cu) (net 4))
 (segment (start 110.255 52.745) (end 116.85 52.745) (width 0.25) (layer F.Cu) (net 4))
 (segment (start 108 77) (end 108 55) (width 0.25) (layer F.Cu) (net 4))
 (segment (start 108 55) (end 110.255 52.745) (width 0.25) (layer F.Cu) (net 4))
 (segment (start 110.38 79.38) (end 108 77) (width 0.25) (layer F.Cu) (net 4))
 (segment (start 110.38 81) (end 110.38 79.38) (width 0.25) (layer F.Cu) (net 4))
 (segment (start 116.85 57.825) (end 113.175 57.825) (width 0.25) (layer F.Cu) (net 8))
 (segment (start 113.175 57.825) (end 112 59) (width 0.25) (layer F.Cu) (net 8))
 (segment (start 112 59) (end 112 73) (width 0.25) (layer F.Cu) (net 8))
 (segment (start 125 81) (end 125 77) (width 0.25) (layer F.Cu) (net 8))
 (segment (start 112 73) (end 114 75) (width 0.25) (layer F.Cu) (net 8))
 (segment (start 114 75) (end 123 75) (width 0.25) (layer F.Cu) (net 8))
 (segment (start 123 75) (end 125 77) (width 0.25) (layer F.Cu) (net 8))
 (segment (start 127.54 76.54) (end 127.54 81) (width 0.25) (layer F.Cu) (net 9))
 (segment (start 125 74) (end 127.54 76.54) (width 0.25) (layer F.Cu) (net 9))
 (segment (start 116.85 59.095) (end 113.905 59.095) (width 0.25) (layer F.Cu) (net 9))
 (segment (start 115 74) (end 125 74) (width 0.25) (layer F.Cu) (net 9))
 (segment (start 113 60) (end 113 72) (width 0.25) (layer F.Cu) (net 9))
 (segment (start 113.905 59.095) (end 113 60) (width 0.25) (layer F.Cu) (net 9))
 (segment (start 113 72) (end 115 74) (width 0.25) (layer F.Cu) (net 9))
 (segment (start 130.08 76.08) (end 130.08 81) (width 0.25) (layer F.Cu) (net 10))
 (segment (start 116.85 60.365) (end 114.635 60.365) (width 0.25) (layer F.Cu) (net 10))
 (segment (start 114 71) (end 116 73) (width 0.25) (layer F.Cu) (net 10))
 (segment (start 114 61) (end 114 71) (width 0.25) (layer F.Cu) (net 10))
 (segment (start 114.635 60.365) (end 114 61) (width 0.25) (layer F.Cu) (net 10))
 (segment (start 130.08 76.08) (end 127 73) (width 0.25) (layer F.Cu) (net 10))
 (segment (start 127 73) (end 116 73) (width 0.25) (layer F.Cu) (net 10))
 (segment (start 116.365 61.635) (end 116.85 61.635) (width 0.25) (layer F.Cu) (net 11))
 (segment (start 115 62) (end 115 70) (width 0.25) (layer F.Cu) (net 11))
 (segment (start 115.365 61.635) (end 115 62) (width 0.25) (layer F.Cu) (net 11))
 (segment (start 116.85 61.635) (end 115.365 61.635) (width 0.25) (layer F.Cu) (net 11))
 (segment (start 117 72) (end 115 70) (width 0.25) (layer F.Cu) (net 11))
 (segment (start 117 72) (end 129 72) (width 0.25) (layer F.Cu) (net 11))
 (segment (start 132.62 75.62) (end 132.62 81) (width 0.25) (layer F.Cu) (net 11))
 (segment (start 129 72) (end 132.62 75.62) (width 0.25) (layer F.Cu) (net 11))
 (segment (start 121 65) (end 119.285 66.715) (width 0.25) (layer F.Cu) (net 13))
 (segment (start 119.285 66.715) (end 116.85 66.715) (width 0.25) (layer F.Cu) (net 13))
 (segment (start 121 52) (end 121 65) (width 0.25) (layer F.Cu) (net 13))
 (segment (start 123 50) (end 121 52) (width 0.25) (layer F.Cu) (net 13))
 (segment (start 134.38 57.38) (end 133 56) (width 0.25) (layer F.Cu) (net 13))
 (segment (start 140 57.38) (end 134.38 57.38) (width 0.25) (layer F.Cu) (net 13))
 (segment (start 133 56) (end 132 55) (width 0.25) (layer F.Cu) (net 13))
 (segment (start 132 55) (end 132 53) (width 0.25) (layer F.Cu) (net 13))
 (segment (start 132 53) (end 132 52) (width 0.25) (layer F.Cu) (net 13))
 (segment (start 132 52) (end 130 50) (width 0.25) (layer F.Cu) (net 13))
 (segment (start 130 50) (end 123 50) (width 0.25) (layer F.Cu) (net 13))
 (segment (start 133.92 59.92) (end 140 59.92) (width 0.25) (layer F.Cu) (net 14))
 (segment (start 129 51) (end 130 52) (width 0.25) (layer F.Cu) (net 14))
 (segment (start 122 53) (end 124 51) (width 0.25) (layer F.Cu) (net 14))
 (segment (start 124 51) (end 129 51) (width 0.25) (layer F.Cu) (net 14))
 (segment (start 130 56) (end 133.92 59.92) (width 0.25) (layer F.Cu) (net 14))
 (segment (start 122 65.97) (end 122 53) (width 0.25) (layer F.Cu) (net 14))
 (segment (start 130 52) (end 130 56) (width 0.25) (layer F.Cu) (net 14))
 (segment (start 119.985 67.985) (end 122 65.97) (width 0.25) (layer F.Cu) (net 14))
 (segment (start 116.85 67.985) (end 119.985 67.985) (width 0.25) (layer F.Cu) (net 14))
 (segment (start 140 62.46) (end 134.46 62.46) (width 0.25) (layer F.Cu) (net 19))
 (segment (start 132.365 60.365) (end 126.15 60.365) (width 0.25) (layer F.Cu) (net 19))
 (segment (start 134.46 62.46) (end 132.365 60.365) (width 0.25) (layer F.Cu) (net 19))
 (segment (start 126.15 61.635) (end 130.635 61.635) (width 0.25) (layer F.Cu) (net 18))
 (segment (start 134 65) (end 140 65) (width 0.25) (layer F.Cu) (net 18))
 (segment (start 130.635 61.635) (end 134 65) (width 0.25) (layer F.Cu) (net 18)))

